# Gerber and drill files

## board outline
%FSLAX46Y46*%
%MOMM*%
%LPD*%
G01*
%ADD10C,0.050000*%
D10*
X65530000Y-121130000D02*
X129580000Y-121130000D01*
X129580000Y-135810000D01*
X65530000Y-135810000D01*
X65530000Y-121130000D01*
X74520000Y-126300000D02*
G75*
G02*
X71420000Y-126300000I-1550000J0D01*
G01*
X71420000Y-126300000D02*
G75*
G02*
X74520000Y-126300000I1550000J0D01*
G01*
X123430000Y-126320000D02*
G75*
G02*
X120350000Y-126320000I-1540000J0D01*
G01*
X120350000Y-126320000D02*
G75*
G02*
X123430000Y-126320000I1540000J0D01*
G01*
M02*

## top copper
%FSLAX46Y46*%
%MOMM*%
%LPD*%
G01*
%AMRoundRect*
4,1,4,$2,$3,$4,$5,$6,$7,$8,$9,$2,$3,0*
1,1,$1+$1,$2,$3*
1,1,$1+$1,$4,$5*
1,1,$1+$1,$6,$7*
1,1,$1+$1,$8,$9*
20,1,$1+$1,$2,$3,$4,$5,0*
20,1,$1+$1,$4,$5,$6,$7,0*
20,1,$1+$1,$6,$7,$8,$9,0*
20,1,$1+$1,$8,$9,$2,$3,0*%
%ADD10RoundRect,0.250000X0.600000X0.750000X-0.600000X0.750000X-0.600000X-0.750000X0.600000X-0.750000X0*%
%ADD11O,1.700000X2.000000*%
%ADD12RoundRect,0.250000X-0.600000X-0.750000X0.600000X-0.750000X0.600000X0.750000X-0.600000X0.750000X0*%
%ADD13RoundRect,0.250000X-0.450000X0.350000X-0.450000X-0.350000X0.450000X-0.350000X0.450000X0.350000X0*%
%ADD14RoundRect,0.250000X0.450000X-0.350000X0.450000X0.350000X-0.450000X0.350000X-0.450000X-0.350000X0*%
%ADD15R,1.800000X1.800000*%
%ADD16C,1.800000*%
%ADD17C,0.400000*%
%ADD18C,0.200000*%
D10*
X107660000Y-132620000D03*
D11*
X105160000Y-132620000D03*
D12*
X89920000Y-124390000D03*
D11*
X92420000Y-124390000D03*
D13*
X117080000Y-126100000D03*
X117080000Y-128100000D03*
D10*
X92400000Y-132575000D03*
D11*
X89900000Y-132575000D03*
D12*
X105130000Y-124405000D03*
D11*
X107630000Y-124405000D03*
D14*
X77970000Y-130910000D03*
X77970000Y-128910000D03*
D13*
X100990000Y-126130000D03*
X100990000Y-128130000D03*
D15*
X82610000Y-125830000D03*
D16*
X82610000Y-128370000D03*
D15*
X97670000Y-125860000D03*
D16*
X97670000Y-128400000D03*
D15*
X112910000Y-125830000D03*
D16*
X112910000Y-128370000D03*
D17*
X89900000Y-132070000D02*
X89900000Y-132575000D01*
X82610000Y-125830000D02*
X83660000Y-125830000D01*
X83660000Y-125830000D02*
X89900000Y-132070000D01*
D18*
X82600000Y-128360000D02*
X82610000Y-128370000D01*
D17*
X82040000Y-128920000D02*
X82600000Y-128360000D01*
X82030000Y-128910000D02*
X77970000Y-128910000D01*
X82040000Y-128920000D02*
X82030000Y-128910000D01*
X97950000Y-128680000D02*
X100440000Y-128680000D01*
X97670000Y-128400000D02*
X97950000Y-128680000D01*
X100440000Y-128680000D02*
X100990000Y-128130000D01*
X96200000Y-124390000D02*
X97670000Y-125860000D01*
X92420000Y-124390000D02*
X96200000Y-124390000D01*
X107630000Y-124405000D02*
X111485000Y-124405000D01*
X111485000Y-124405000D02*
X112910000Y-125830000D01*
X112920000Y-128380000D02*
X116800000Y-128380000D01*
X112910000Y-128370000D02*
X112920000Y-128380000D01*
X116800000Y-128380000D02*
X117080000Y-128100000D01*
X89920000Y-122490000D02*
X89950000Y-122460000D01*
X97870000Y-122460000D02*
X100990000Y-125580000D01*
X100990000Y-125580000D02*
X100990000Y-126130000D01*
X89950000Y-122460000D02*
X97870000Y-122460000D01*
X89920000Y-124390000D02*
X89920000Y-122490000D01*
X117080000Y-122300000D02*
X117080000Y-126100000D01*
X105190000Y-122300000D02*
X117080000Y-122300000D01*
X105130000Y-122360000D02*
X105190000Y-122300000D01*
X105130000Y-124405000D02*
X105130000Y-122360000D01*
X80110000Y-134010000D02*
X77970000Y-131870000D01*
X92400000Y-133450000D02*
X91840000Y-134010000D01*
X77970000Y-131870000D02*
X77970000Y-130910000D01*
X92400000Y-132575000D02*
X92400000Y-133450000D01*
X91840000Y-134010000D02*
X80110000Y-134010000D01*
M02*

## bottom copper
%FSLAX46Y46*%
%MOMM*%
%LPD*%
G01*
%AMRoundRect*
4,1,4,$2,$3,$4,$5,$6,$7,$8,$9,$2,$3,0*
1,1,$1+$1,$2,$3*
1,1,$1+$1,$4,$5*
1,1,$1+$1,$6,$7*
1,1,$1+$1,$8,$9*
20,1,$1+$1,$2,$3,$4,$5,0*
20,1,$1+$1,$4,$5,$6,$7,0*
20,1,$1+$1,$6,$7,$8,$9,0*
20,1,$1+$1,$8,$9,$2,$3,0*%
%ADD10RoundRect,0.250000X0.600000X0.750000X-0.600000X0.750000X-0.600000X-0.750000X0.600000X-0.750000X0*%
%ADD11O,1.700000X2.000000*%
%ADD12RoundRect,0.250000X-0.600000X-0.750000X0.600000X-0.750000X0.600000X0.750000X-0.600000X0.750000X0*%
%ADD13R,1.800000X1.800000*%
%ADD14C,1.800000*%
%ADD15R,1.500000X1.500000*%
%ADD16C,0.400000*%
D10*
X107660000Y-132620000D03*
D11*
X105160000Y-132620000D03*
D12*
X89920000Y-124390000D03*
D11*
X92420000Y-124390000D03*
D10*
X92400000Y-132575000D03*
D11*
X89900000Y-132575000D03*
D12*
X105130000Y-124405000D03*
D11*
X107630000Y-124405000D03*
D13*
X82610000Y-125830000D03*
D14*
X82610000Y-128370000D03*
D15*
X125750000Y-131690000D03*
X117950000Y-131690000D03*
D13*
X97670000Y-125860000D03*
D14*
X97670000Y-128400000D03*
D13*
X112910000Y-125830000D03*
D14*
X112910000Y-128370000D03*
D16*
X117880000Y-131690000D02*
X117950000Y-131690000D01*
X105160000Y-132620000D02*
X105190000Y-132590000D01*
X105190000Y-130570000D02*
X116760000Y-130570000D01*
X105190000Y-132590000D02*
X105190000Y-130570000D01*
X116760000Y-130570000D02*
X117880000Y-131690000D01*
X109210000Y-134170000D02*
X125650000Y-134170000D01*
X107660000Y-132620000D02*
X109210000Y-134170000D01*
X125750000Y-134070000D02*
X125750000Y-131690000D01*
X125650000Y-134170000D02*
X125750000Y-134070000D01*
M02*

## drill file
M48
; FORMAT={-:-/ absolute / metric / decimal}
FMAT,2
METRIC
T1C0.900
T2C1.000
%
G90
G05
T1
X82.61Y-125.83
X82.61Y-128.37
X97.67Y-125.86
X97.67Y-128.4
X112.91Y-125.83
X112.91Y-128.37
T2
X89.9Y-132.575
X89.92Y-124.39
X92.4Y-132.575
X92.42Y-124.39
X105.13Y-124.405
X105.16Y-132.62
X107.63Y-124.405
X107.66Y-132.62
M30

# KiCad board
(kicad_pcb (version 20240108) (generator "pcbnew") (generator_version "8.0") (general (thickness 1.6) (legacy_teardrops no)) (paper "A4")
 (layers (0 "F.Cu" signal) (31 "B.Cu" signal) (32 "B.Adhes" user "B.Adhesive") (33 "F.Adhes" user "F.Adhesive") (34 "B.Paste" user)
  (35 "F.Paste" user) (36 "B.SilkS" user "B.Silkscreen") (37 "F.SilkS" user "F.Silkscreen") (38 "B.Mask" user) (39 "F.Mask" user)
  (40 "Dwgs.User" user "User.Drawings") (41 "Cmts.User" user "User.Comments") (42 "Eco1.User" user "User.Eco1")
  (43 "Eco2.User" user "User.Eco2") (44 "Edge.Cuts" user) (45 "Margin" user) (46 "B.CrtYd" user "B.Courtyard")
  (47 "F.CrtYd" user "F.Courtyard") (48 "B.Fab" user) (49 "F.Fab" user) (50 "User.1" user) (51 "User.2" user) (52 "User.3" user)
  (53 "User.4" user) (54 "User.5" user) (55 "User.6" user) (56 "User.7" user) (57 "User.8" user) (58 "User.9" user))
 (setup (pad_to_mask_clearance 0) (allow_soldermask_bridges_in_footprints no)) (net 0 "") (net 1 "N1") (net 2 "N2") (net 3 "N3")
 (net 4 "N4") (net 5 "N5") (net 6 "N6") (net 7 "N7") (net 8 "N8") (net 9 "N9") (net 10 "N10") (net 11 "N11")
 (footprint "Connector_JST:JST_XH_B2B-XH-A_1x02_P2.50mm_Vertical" (layer "F.Cu") (at 107.66 132.62 180)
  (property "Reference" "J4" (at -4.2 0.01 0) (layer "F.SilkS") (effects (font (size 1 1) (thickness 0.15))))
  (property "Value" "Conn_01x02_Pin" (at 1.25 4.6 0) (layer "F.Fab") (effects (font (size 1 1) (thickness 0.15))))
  (pad "1" thru_hole roundrect (at 0 0 180) (size 1.7 2) (drill 1) (layers "*.Cu" "*.Mask") (remove_unused_layers no)
   (roundrect_rratio 0.147059) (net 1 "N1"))
  (pad "2" thru_hole oval (at 2.5 0 180) (size 1.7 2) (drill 1) (layers "*.Cu" "*.Mask") (remove_unused_layers no) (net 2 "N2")))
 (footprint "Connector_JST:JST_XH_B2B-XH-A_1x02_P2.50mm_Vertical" (layer "F.Cu") (at 89.92 124.39)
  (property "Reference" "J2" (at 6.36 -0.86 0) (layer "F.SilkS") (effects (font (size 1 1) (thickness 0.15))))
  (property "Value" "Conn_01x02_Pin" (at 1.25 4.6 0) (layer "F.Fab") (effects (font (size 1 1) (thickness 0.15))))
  (pad "1" thru_hole roundrect (at 0 0) (size 1.7 2) (drill 1) (layers "*.Cu" "*.Mask") (remove_unused_layers no)
   (roundrect_rratio 0.147059) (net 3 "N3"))
  (pad "2" thru_hole oval (at 2.5 0) (size 1.7 2) (drill 1) (layers "*.Cu" "*.Mask") (remove_unused_layers no) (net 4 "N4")))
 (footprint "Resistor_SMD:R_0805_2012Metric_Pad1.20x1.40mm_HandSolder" (layer "F.Cu") (at 117.08 127.1 -90)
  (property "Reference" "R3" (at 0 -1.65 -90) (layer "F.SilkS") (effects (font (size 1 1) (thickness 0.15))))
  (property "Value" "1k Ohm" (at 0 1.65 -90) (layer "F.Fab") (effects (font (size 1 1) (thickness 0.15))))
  (pad "1" smd roundrect (at -1 0 270) (size 1.2 1.4) (layers "F.Cu" "F.Paste" "F.Mask") (roundrect_rratio 0.208333) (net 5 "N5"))
  (pad "2" smd roundrect (at 1 0 270) (size 1.2 1.4) (layers "F.Cu" "F.Paste" "F.Mask") (roundrect_rratio 0.208333) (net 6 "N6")))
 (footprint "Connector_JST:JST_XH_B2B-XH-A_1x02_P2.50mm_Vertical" (layer "F.Cu") (at 92.4 132.575 180)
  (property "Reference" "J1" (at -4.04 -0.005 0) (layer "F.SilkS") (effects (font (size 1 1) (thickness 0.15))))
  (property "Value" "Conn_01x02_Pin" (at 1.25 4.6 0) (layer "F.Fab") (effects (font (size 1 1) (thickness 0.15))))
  (pad "1" thru_hole roundrect (at 0 0 180) (size 1.7 2) (drill 1) (layers "*.Cu" "*.Mask") (remove_unused_layers no)
   (roundrect_rratio 0.147059) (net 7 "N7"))
  (pad "2" thru_hole oval (at 2.5 0 180) (size 1.7 2) (drill 1) (layers "*.Cu" "*.Mask") (remove_unused_layers no) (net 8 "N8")))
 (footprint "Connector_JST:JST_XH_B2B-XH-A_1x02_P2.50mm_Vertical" (layer "F.Cu") (at 105.13 124.405)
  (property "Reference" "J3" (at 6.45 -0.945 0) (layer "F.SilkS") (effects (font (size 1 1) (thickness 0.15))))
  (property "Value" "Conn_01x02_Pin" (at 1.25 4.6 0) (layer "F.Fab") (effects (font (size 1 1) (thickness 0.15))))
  (pad "1" thru_hole roundrect (at 0 0) (size 1.7 2) (drill 1) (layers "*.Cu" "*.Mask") (remove_unused_layers no)
   (roundrect_rratio 0.147059) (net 5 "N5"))
  (pad "2" thru_hole oval (at 2.5 0) (size 1.7 2) (drill 1) (layers "*.Cu" "*.Mask") (remove_unused_layers no) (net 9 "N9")))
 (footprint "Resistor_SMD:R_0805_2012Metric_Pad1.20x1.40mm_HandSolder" (layer "F.Cu") (at 77.97 129.91 90)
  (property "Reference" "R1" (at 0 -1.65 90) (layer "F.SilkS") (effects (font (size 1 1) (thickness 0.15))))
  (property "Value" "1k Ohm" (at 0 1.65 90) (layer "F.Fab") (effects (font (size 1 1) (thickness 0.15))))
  (pad "1" smd roundrect (at -1 0 90) (size 1.2 1.4) (layers "F.Cu" "F.Paste" "F.Mask") (roundrect_rratio 0.208333) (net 7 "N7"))
  (pad "2" smd roundrect (at 1 0 90) (size 1.2 1.4) (layers "F.Cu" "F.Paste" "F.Mask") (roundrect_rratio 0.208333) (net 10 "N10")))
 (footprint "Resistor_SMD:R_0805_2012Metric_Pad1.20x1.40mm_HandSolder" (layer "F.Cu") (at 100.99 127.13 -90)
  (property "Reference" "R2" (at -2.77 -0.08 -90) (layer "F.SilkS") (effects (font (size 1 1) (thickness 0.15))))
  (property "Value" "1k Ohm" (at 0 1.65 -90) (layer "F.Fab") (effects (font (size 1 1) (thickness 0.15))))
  (pad "1" smd roundrect (at -1 0 270) (size 1.2 1.4) (layers "F.Cu" "F.Paste" "F.Mask") (roundrect_rratio 0.208333) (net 3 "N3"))
  (pad "2" smd roundrect (at 1 0 270) (size 1.2 1.4) (layers "F.Cu" "F.Paste" "F.Mask") (roundrect_rratio 0.208333) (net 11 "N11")))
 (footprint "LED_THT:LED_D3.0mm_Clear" (layer "B.Cu") (at 82.61 125.83 -90)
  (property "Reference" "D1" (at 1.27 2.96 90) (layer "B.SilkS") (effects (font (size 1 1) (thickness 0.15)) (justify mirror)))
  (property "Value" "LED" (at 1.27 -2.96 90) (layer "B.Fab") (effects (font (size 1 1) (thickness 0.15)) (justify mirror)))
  (pad "1" thru_hole rect (at 0 0 270) (size 1.8 1.8) (drill 0.9) (layers "*.Cu" "*.Mask") (remove_unused_layers no) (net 8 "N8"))
  (pad "2" thru_hole circle (at 2.54 0 270) (size 1.8 1.8) (drill 0.9) (layers "*.Cu" "*.Mask") (remove_unused_layers no) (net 10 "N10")))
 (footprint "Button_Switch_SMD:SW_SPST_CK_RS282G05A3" (layer "B.Cu") (at 121.85 131.69 180)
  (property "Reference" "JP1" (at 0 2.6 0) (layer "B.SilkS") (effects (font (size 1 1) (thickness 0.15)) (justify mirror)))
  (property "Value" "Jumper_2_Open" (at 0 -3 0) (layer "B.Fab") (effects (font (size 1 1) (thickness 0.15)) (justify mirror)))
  (pad "1" smd rect (at -3.9 0 180) (size 1.5 1.5) (layers "B.Cu" "B.Paste" "B.Mask") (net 1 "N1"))
  (pad "2" smd rect (at 3.9 0 180) (size 1.5 1.5) (layers "B.Cu" "B.Paste" "B.Mask") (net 2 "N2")))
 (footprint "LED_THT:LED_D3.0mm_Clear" (layer "B.Cu") (at 97.67 125.86 -90)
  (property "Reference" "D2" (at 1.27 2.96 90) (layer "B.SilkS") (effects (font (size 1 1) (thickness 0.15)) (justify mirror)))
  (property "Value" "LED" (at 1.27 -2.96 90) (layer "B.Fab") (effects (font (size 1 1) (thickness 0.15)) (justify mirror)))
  (pad "1" thru_hole rect (at 0 0 270) (size 1.8 1.8) (drill 0.9) (layers "*.Cu" "*.Mask") (remove_unused_layers no) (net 4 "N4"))
  (pad "2" thru_hole circle (at 2.54 0 270) (size 1.8 1.8) (drill 0.9) (layers "*.Cu" "*.Mask") (remove_unused_layers no) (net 11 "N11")))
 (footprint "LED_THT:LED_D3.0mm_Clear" (layer "B.Cu") (at 112.91 125.83 -90)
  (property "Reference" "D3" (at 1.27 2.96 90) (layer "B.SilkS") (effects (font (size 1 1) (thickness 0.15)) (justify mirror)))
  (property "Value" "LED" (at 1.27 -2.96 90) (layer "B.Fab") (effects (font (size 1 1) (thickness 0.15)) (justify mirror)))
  (pad "1" thru_hole rect (at 0 0 270) (size 1.8 1.8) (drill 0.9) (layers "*.Cu" "*.Mask") (remove_unused_layers no) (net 9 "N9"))
  (pad "2" thru_hole circle (at 2.54 0 270) (size 1.8 1.8) (drill 0.9) (layers "*.Cu" "*.Mask") (remove_unused_layers no) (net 6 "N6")))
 (gr_rect (start 65.53 121.13) (end 129.58 135.81) (stroke (width 0.05) (type default)) (fill none) (layer "Edge.Cuts"))
 (gr_circle (center 72.97 126.3) (end 74.52 126.3) (stroke (width 0.05) (type default)) (fill none) (layer "Edge.Cuts"))
 (gr_circle (center 121.89 126.32) (end 123.43 126.32) (stroke (width 0.05) (type default)) (fill none) (layer "Edge.Cuts"))
 (segment (start 89.9 132.07) (end 89.9 132.575) (width 0.4) (layer "F.Cu") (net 8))
 (segment (start 82.61 125.83) (end 83.66 125.83) (width 0.4) (layer "F.Cu") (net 8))
 (segment (start 83.66 125.83) (end 89.9 132.07) (width 0.4) (layer "F.Cu") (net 8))
 (segment (start 82.6 128.36) (end 82.61 128.37) (width 0.2) (layer "F.Cu") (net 10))
 (segment (start 82.04 128.92) (end 82.6 128.36) (width 0.4) (layer "F.Cu") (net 10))
 (segment (start 82.03 128.91) (end 77.97 128.91) (width 0.4) (layer "F.Cu") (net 10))
 (segment (start 82.04 128.92) (end 82.03 128.91) (width 0.4) (layer "F.Cu") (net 10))
 (segment (start 97.95 128.68) (end 100.44 128.68) (width 0.4) (layer "F.Cu") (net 11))
 (segment (start 97.67 128.4) (end 97.95 128.68) (width 0.4) (layer "F.Cu") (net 11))
 (segment (start 100.44 128.68) (end 100.99 128.13) (width 0.4) (layer "F.Cu") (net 11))
 (segment (start 96.2 124.39) (end 97.67 125.86) (width 0.4) (layer "F.Cu") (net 4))
 (segment (start 92.42 124.39) (end 96.2 124.39) (width 0.4) (layer "F.Cu") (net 4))
 (segment (start 107.63 124.405) (end 111.485 124.405) (width 0.4) (layer "F.Cu") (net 9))
 (segment (start 111.485 124.405) (end 112.91 125.83) (width 0.4) (layer "F.Cu") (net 9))
 (segment (start 112.92 128.38) (end 116.8 128.38) (width 0.4) (layer "F.Cu") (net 6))
 (segment (start 112.91 128.37) (end 112.92 128.38) (width 0.4) (layer "F.Cu") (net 6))
 (segment (start 116.8 128.38) (end 117.08 128.1) (width 0.4) (layer "F.Cu") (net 6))
 (segment (start 89.92 122.49) (end 89.95 122.46) (width 0.4) (layer "F.Cu") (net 3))
 (segment (start 97.87 122.46) (end 100.99 125.58) (width 0.4) (layer "F.Cu") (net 3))
 (segment (start 100.99 125.58) (end 100.99 126.13) (width 0.4) (layer "F.Cu") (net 3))
 (segment (start 89.95 122.46) (end 97.87 122.46) (width 0.4) (layer "F.Cu") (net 3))
 (segment (start 89.92 124.39) (end 89.92 122.49) (width 0.4) (layer "F.Cu") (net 3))
 (segment (start 117.08 122.3) (end 117.08 126.1) (width 0.4) (layer "F.Cu") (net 5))
 (segment (start 105.19 122.3) (end 117.08 122.3) (width 0.4) (layer "F.Cu") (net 5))
 (segment (start 105.13 122.36) (end 105.19 122.3) (width 0.4) (layer "F.Cu") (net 5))
 (segment (start 105.13 124.405) (end 105.13 122.36) (width 0.4) (layer "F.Cu") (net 5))
 (segment (start 117.88 131.69) (end 117.95 131.69) (width 0.4) (layer "B.Cu") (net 2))
 (segment (start 105.16 132.62) (end 105.19 132.59) (width 0.4) (layer "B.Cu") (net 2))
 (segment (start 105.19 130.57) (end 116.76 130.57) (width 0.4) (layer "B.Cu") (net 2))
 (segment (start 105.19 132.59) (end 105.19 130.57) (width 0.4) (layer "B.Cu") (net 2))
 (segment (start 116.76 130.57) (end 117.88 131.69) (width 0.4) (layer "B.Cu") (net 2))
 (segment (start 109.21 134.17) (end 125.65 134.17) (width 0.4) (layer "B.Cu") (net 1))
 (segment (start 107.66 132.62) (end 109.21 134.17) (width 0.4) (layer "B.Cu") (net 1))
 (segment (start 125.75 134.07) (end 125.75 131.69) (width 0.4) (layer "B.Cu") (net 1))
 (segment (start 125.65 134.17) (end 125.75 134.07) (width 0.4) (layer "B.Cu") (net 1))
 (segment (start 80.11 134.01) (end 77.97 131.87) (width 0.4) (layer "F.Cu") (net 7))
 (segment (start 92.4 133.45) (end 91.84 134.01) (width 0.4) (layer "F.Cu") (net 7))
 (segment (start 77.97 131.87) (end 77.97 130.91) (width 0.4) (layer "F.Cu") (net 7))
 (segment (start 92.4 132.575) (end 92.4 133.45) (width 0.4) (layer "F.Cu") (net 7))
 (segment (start 91.84 134.01) (end 80.11 134.01) (width 0.4) (layer "F.Cu") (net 7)))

